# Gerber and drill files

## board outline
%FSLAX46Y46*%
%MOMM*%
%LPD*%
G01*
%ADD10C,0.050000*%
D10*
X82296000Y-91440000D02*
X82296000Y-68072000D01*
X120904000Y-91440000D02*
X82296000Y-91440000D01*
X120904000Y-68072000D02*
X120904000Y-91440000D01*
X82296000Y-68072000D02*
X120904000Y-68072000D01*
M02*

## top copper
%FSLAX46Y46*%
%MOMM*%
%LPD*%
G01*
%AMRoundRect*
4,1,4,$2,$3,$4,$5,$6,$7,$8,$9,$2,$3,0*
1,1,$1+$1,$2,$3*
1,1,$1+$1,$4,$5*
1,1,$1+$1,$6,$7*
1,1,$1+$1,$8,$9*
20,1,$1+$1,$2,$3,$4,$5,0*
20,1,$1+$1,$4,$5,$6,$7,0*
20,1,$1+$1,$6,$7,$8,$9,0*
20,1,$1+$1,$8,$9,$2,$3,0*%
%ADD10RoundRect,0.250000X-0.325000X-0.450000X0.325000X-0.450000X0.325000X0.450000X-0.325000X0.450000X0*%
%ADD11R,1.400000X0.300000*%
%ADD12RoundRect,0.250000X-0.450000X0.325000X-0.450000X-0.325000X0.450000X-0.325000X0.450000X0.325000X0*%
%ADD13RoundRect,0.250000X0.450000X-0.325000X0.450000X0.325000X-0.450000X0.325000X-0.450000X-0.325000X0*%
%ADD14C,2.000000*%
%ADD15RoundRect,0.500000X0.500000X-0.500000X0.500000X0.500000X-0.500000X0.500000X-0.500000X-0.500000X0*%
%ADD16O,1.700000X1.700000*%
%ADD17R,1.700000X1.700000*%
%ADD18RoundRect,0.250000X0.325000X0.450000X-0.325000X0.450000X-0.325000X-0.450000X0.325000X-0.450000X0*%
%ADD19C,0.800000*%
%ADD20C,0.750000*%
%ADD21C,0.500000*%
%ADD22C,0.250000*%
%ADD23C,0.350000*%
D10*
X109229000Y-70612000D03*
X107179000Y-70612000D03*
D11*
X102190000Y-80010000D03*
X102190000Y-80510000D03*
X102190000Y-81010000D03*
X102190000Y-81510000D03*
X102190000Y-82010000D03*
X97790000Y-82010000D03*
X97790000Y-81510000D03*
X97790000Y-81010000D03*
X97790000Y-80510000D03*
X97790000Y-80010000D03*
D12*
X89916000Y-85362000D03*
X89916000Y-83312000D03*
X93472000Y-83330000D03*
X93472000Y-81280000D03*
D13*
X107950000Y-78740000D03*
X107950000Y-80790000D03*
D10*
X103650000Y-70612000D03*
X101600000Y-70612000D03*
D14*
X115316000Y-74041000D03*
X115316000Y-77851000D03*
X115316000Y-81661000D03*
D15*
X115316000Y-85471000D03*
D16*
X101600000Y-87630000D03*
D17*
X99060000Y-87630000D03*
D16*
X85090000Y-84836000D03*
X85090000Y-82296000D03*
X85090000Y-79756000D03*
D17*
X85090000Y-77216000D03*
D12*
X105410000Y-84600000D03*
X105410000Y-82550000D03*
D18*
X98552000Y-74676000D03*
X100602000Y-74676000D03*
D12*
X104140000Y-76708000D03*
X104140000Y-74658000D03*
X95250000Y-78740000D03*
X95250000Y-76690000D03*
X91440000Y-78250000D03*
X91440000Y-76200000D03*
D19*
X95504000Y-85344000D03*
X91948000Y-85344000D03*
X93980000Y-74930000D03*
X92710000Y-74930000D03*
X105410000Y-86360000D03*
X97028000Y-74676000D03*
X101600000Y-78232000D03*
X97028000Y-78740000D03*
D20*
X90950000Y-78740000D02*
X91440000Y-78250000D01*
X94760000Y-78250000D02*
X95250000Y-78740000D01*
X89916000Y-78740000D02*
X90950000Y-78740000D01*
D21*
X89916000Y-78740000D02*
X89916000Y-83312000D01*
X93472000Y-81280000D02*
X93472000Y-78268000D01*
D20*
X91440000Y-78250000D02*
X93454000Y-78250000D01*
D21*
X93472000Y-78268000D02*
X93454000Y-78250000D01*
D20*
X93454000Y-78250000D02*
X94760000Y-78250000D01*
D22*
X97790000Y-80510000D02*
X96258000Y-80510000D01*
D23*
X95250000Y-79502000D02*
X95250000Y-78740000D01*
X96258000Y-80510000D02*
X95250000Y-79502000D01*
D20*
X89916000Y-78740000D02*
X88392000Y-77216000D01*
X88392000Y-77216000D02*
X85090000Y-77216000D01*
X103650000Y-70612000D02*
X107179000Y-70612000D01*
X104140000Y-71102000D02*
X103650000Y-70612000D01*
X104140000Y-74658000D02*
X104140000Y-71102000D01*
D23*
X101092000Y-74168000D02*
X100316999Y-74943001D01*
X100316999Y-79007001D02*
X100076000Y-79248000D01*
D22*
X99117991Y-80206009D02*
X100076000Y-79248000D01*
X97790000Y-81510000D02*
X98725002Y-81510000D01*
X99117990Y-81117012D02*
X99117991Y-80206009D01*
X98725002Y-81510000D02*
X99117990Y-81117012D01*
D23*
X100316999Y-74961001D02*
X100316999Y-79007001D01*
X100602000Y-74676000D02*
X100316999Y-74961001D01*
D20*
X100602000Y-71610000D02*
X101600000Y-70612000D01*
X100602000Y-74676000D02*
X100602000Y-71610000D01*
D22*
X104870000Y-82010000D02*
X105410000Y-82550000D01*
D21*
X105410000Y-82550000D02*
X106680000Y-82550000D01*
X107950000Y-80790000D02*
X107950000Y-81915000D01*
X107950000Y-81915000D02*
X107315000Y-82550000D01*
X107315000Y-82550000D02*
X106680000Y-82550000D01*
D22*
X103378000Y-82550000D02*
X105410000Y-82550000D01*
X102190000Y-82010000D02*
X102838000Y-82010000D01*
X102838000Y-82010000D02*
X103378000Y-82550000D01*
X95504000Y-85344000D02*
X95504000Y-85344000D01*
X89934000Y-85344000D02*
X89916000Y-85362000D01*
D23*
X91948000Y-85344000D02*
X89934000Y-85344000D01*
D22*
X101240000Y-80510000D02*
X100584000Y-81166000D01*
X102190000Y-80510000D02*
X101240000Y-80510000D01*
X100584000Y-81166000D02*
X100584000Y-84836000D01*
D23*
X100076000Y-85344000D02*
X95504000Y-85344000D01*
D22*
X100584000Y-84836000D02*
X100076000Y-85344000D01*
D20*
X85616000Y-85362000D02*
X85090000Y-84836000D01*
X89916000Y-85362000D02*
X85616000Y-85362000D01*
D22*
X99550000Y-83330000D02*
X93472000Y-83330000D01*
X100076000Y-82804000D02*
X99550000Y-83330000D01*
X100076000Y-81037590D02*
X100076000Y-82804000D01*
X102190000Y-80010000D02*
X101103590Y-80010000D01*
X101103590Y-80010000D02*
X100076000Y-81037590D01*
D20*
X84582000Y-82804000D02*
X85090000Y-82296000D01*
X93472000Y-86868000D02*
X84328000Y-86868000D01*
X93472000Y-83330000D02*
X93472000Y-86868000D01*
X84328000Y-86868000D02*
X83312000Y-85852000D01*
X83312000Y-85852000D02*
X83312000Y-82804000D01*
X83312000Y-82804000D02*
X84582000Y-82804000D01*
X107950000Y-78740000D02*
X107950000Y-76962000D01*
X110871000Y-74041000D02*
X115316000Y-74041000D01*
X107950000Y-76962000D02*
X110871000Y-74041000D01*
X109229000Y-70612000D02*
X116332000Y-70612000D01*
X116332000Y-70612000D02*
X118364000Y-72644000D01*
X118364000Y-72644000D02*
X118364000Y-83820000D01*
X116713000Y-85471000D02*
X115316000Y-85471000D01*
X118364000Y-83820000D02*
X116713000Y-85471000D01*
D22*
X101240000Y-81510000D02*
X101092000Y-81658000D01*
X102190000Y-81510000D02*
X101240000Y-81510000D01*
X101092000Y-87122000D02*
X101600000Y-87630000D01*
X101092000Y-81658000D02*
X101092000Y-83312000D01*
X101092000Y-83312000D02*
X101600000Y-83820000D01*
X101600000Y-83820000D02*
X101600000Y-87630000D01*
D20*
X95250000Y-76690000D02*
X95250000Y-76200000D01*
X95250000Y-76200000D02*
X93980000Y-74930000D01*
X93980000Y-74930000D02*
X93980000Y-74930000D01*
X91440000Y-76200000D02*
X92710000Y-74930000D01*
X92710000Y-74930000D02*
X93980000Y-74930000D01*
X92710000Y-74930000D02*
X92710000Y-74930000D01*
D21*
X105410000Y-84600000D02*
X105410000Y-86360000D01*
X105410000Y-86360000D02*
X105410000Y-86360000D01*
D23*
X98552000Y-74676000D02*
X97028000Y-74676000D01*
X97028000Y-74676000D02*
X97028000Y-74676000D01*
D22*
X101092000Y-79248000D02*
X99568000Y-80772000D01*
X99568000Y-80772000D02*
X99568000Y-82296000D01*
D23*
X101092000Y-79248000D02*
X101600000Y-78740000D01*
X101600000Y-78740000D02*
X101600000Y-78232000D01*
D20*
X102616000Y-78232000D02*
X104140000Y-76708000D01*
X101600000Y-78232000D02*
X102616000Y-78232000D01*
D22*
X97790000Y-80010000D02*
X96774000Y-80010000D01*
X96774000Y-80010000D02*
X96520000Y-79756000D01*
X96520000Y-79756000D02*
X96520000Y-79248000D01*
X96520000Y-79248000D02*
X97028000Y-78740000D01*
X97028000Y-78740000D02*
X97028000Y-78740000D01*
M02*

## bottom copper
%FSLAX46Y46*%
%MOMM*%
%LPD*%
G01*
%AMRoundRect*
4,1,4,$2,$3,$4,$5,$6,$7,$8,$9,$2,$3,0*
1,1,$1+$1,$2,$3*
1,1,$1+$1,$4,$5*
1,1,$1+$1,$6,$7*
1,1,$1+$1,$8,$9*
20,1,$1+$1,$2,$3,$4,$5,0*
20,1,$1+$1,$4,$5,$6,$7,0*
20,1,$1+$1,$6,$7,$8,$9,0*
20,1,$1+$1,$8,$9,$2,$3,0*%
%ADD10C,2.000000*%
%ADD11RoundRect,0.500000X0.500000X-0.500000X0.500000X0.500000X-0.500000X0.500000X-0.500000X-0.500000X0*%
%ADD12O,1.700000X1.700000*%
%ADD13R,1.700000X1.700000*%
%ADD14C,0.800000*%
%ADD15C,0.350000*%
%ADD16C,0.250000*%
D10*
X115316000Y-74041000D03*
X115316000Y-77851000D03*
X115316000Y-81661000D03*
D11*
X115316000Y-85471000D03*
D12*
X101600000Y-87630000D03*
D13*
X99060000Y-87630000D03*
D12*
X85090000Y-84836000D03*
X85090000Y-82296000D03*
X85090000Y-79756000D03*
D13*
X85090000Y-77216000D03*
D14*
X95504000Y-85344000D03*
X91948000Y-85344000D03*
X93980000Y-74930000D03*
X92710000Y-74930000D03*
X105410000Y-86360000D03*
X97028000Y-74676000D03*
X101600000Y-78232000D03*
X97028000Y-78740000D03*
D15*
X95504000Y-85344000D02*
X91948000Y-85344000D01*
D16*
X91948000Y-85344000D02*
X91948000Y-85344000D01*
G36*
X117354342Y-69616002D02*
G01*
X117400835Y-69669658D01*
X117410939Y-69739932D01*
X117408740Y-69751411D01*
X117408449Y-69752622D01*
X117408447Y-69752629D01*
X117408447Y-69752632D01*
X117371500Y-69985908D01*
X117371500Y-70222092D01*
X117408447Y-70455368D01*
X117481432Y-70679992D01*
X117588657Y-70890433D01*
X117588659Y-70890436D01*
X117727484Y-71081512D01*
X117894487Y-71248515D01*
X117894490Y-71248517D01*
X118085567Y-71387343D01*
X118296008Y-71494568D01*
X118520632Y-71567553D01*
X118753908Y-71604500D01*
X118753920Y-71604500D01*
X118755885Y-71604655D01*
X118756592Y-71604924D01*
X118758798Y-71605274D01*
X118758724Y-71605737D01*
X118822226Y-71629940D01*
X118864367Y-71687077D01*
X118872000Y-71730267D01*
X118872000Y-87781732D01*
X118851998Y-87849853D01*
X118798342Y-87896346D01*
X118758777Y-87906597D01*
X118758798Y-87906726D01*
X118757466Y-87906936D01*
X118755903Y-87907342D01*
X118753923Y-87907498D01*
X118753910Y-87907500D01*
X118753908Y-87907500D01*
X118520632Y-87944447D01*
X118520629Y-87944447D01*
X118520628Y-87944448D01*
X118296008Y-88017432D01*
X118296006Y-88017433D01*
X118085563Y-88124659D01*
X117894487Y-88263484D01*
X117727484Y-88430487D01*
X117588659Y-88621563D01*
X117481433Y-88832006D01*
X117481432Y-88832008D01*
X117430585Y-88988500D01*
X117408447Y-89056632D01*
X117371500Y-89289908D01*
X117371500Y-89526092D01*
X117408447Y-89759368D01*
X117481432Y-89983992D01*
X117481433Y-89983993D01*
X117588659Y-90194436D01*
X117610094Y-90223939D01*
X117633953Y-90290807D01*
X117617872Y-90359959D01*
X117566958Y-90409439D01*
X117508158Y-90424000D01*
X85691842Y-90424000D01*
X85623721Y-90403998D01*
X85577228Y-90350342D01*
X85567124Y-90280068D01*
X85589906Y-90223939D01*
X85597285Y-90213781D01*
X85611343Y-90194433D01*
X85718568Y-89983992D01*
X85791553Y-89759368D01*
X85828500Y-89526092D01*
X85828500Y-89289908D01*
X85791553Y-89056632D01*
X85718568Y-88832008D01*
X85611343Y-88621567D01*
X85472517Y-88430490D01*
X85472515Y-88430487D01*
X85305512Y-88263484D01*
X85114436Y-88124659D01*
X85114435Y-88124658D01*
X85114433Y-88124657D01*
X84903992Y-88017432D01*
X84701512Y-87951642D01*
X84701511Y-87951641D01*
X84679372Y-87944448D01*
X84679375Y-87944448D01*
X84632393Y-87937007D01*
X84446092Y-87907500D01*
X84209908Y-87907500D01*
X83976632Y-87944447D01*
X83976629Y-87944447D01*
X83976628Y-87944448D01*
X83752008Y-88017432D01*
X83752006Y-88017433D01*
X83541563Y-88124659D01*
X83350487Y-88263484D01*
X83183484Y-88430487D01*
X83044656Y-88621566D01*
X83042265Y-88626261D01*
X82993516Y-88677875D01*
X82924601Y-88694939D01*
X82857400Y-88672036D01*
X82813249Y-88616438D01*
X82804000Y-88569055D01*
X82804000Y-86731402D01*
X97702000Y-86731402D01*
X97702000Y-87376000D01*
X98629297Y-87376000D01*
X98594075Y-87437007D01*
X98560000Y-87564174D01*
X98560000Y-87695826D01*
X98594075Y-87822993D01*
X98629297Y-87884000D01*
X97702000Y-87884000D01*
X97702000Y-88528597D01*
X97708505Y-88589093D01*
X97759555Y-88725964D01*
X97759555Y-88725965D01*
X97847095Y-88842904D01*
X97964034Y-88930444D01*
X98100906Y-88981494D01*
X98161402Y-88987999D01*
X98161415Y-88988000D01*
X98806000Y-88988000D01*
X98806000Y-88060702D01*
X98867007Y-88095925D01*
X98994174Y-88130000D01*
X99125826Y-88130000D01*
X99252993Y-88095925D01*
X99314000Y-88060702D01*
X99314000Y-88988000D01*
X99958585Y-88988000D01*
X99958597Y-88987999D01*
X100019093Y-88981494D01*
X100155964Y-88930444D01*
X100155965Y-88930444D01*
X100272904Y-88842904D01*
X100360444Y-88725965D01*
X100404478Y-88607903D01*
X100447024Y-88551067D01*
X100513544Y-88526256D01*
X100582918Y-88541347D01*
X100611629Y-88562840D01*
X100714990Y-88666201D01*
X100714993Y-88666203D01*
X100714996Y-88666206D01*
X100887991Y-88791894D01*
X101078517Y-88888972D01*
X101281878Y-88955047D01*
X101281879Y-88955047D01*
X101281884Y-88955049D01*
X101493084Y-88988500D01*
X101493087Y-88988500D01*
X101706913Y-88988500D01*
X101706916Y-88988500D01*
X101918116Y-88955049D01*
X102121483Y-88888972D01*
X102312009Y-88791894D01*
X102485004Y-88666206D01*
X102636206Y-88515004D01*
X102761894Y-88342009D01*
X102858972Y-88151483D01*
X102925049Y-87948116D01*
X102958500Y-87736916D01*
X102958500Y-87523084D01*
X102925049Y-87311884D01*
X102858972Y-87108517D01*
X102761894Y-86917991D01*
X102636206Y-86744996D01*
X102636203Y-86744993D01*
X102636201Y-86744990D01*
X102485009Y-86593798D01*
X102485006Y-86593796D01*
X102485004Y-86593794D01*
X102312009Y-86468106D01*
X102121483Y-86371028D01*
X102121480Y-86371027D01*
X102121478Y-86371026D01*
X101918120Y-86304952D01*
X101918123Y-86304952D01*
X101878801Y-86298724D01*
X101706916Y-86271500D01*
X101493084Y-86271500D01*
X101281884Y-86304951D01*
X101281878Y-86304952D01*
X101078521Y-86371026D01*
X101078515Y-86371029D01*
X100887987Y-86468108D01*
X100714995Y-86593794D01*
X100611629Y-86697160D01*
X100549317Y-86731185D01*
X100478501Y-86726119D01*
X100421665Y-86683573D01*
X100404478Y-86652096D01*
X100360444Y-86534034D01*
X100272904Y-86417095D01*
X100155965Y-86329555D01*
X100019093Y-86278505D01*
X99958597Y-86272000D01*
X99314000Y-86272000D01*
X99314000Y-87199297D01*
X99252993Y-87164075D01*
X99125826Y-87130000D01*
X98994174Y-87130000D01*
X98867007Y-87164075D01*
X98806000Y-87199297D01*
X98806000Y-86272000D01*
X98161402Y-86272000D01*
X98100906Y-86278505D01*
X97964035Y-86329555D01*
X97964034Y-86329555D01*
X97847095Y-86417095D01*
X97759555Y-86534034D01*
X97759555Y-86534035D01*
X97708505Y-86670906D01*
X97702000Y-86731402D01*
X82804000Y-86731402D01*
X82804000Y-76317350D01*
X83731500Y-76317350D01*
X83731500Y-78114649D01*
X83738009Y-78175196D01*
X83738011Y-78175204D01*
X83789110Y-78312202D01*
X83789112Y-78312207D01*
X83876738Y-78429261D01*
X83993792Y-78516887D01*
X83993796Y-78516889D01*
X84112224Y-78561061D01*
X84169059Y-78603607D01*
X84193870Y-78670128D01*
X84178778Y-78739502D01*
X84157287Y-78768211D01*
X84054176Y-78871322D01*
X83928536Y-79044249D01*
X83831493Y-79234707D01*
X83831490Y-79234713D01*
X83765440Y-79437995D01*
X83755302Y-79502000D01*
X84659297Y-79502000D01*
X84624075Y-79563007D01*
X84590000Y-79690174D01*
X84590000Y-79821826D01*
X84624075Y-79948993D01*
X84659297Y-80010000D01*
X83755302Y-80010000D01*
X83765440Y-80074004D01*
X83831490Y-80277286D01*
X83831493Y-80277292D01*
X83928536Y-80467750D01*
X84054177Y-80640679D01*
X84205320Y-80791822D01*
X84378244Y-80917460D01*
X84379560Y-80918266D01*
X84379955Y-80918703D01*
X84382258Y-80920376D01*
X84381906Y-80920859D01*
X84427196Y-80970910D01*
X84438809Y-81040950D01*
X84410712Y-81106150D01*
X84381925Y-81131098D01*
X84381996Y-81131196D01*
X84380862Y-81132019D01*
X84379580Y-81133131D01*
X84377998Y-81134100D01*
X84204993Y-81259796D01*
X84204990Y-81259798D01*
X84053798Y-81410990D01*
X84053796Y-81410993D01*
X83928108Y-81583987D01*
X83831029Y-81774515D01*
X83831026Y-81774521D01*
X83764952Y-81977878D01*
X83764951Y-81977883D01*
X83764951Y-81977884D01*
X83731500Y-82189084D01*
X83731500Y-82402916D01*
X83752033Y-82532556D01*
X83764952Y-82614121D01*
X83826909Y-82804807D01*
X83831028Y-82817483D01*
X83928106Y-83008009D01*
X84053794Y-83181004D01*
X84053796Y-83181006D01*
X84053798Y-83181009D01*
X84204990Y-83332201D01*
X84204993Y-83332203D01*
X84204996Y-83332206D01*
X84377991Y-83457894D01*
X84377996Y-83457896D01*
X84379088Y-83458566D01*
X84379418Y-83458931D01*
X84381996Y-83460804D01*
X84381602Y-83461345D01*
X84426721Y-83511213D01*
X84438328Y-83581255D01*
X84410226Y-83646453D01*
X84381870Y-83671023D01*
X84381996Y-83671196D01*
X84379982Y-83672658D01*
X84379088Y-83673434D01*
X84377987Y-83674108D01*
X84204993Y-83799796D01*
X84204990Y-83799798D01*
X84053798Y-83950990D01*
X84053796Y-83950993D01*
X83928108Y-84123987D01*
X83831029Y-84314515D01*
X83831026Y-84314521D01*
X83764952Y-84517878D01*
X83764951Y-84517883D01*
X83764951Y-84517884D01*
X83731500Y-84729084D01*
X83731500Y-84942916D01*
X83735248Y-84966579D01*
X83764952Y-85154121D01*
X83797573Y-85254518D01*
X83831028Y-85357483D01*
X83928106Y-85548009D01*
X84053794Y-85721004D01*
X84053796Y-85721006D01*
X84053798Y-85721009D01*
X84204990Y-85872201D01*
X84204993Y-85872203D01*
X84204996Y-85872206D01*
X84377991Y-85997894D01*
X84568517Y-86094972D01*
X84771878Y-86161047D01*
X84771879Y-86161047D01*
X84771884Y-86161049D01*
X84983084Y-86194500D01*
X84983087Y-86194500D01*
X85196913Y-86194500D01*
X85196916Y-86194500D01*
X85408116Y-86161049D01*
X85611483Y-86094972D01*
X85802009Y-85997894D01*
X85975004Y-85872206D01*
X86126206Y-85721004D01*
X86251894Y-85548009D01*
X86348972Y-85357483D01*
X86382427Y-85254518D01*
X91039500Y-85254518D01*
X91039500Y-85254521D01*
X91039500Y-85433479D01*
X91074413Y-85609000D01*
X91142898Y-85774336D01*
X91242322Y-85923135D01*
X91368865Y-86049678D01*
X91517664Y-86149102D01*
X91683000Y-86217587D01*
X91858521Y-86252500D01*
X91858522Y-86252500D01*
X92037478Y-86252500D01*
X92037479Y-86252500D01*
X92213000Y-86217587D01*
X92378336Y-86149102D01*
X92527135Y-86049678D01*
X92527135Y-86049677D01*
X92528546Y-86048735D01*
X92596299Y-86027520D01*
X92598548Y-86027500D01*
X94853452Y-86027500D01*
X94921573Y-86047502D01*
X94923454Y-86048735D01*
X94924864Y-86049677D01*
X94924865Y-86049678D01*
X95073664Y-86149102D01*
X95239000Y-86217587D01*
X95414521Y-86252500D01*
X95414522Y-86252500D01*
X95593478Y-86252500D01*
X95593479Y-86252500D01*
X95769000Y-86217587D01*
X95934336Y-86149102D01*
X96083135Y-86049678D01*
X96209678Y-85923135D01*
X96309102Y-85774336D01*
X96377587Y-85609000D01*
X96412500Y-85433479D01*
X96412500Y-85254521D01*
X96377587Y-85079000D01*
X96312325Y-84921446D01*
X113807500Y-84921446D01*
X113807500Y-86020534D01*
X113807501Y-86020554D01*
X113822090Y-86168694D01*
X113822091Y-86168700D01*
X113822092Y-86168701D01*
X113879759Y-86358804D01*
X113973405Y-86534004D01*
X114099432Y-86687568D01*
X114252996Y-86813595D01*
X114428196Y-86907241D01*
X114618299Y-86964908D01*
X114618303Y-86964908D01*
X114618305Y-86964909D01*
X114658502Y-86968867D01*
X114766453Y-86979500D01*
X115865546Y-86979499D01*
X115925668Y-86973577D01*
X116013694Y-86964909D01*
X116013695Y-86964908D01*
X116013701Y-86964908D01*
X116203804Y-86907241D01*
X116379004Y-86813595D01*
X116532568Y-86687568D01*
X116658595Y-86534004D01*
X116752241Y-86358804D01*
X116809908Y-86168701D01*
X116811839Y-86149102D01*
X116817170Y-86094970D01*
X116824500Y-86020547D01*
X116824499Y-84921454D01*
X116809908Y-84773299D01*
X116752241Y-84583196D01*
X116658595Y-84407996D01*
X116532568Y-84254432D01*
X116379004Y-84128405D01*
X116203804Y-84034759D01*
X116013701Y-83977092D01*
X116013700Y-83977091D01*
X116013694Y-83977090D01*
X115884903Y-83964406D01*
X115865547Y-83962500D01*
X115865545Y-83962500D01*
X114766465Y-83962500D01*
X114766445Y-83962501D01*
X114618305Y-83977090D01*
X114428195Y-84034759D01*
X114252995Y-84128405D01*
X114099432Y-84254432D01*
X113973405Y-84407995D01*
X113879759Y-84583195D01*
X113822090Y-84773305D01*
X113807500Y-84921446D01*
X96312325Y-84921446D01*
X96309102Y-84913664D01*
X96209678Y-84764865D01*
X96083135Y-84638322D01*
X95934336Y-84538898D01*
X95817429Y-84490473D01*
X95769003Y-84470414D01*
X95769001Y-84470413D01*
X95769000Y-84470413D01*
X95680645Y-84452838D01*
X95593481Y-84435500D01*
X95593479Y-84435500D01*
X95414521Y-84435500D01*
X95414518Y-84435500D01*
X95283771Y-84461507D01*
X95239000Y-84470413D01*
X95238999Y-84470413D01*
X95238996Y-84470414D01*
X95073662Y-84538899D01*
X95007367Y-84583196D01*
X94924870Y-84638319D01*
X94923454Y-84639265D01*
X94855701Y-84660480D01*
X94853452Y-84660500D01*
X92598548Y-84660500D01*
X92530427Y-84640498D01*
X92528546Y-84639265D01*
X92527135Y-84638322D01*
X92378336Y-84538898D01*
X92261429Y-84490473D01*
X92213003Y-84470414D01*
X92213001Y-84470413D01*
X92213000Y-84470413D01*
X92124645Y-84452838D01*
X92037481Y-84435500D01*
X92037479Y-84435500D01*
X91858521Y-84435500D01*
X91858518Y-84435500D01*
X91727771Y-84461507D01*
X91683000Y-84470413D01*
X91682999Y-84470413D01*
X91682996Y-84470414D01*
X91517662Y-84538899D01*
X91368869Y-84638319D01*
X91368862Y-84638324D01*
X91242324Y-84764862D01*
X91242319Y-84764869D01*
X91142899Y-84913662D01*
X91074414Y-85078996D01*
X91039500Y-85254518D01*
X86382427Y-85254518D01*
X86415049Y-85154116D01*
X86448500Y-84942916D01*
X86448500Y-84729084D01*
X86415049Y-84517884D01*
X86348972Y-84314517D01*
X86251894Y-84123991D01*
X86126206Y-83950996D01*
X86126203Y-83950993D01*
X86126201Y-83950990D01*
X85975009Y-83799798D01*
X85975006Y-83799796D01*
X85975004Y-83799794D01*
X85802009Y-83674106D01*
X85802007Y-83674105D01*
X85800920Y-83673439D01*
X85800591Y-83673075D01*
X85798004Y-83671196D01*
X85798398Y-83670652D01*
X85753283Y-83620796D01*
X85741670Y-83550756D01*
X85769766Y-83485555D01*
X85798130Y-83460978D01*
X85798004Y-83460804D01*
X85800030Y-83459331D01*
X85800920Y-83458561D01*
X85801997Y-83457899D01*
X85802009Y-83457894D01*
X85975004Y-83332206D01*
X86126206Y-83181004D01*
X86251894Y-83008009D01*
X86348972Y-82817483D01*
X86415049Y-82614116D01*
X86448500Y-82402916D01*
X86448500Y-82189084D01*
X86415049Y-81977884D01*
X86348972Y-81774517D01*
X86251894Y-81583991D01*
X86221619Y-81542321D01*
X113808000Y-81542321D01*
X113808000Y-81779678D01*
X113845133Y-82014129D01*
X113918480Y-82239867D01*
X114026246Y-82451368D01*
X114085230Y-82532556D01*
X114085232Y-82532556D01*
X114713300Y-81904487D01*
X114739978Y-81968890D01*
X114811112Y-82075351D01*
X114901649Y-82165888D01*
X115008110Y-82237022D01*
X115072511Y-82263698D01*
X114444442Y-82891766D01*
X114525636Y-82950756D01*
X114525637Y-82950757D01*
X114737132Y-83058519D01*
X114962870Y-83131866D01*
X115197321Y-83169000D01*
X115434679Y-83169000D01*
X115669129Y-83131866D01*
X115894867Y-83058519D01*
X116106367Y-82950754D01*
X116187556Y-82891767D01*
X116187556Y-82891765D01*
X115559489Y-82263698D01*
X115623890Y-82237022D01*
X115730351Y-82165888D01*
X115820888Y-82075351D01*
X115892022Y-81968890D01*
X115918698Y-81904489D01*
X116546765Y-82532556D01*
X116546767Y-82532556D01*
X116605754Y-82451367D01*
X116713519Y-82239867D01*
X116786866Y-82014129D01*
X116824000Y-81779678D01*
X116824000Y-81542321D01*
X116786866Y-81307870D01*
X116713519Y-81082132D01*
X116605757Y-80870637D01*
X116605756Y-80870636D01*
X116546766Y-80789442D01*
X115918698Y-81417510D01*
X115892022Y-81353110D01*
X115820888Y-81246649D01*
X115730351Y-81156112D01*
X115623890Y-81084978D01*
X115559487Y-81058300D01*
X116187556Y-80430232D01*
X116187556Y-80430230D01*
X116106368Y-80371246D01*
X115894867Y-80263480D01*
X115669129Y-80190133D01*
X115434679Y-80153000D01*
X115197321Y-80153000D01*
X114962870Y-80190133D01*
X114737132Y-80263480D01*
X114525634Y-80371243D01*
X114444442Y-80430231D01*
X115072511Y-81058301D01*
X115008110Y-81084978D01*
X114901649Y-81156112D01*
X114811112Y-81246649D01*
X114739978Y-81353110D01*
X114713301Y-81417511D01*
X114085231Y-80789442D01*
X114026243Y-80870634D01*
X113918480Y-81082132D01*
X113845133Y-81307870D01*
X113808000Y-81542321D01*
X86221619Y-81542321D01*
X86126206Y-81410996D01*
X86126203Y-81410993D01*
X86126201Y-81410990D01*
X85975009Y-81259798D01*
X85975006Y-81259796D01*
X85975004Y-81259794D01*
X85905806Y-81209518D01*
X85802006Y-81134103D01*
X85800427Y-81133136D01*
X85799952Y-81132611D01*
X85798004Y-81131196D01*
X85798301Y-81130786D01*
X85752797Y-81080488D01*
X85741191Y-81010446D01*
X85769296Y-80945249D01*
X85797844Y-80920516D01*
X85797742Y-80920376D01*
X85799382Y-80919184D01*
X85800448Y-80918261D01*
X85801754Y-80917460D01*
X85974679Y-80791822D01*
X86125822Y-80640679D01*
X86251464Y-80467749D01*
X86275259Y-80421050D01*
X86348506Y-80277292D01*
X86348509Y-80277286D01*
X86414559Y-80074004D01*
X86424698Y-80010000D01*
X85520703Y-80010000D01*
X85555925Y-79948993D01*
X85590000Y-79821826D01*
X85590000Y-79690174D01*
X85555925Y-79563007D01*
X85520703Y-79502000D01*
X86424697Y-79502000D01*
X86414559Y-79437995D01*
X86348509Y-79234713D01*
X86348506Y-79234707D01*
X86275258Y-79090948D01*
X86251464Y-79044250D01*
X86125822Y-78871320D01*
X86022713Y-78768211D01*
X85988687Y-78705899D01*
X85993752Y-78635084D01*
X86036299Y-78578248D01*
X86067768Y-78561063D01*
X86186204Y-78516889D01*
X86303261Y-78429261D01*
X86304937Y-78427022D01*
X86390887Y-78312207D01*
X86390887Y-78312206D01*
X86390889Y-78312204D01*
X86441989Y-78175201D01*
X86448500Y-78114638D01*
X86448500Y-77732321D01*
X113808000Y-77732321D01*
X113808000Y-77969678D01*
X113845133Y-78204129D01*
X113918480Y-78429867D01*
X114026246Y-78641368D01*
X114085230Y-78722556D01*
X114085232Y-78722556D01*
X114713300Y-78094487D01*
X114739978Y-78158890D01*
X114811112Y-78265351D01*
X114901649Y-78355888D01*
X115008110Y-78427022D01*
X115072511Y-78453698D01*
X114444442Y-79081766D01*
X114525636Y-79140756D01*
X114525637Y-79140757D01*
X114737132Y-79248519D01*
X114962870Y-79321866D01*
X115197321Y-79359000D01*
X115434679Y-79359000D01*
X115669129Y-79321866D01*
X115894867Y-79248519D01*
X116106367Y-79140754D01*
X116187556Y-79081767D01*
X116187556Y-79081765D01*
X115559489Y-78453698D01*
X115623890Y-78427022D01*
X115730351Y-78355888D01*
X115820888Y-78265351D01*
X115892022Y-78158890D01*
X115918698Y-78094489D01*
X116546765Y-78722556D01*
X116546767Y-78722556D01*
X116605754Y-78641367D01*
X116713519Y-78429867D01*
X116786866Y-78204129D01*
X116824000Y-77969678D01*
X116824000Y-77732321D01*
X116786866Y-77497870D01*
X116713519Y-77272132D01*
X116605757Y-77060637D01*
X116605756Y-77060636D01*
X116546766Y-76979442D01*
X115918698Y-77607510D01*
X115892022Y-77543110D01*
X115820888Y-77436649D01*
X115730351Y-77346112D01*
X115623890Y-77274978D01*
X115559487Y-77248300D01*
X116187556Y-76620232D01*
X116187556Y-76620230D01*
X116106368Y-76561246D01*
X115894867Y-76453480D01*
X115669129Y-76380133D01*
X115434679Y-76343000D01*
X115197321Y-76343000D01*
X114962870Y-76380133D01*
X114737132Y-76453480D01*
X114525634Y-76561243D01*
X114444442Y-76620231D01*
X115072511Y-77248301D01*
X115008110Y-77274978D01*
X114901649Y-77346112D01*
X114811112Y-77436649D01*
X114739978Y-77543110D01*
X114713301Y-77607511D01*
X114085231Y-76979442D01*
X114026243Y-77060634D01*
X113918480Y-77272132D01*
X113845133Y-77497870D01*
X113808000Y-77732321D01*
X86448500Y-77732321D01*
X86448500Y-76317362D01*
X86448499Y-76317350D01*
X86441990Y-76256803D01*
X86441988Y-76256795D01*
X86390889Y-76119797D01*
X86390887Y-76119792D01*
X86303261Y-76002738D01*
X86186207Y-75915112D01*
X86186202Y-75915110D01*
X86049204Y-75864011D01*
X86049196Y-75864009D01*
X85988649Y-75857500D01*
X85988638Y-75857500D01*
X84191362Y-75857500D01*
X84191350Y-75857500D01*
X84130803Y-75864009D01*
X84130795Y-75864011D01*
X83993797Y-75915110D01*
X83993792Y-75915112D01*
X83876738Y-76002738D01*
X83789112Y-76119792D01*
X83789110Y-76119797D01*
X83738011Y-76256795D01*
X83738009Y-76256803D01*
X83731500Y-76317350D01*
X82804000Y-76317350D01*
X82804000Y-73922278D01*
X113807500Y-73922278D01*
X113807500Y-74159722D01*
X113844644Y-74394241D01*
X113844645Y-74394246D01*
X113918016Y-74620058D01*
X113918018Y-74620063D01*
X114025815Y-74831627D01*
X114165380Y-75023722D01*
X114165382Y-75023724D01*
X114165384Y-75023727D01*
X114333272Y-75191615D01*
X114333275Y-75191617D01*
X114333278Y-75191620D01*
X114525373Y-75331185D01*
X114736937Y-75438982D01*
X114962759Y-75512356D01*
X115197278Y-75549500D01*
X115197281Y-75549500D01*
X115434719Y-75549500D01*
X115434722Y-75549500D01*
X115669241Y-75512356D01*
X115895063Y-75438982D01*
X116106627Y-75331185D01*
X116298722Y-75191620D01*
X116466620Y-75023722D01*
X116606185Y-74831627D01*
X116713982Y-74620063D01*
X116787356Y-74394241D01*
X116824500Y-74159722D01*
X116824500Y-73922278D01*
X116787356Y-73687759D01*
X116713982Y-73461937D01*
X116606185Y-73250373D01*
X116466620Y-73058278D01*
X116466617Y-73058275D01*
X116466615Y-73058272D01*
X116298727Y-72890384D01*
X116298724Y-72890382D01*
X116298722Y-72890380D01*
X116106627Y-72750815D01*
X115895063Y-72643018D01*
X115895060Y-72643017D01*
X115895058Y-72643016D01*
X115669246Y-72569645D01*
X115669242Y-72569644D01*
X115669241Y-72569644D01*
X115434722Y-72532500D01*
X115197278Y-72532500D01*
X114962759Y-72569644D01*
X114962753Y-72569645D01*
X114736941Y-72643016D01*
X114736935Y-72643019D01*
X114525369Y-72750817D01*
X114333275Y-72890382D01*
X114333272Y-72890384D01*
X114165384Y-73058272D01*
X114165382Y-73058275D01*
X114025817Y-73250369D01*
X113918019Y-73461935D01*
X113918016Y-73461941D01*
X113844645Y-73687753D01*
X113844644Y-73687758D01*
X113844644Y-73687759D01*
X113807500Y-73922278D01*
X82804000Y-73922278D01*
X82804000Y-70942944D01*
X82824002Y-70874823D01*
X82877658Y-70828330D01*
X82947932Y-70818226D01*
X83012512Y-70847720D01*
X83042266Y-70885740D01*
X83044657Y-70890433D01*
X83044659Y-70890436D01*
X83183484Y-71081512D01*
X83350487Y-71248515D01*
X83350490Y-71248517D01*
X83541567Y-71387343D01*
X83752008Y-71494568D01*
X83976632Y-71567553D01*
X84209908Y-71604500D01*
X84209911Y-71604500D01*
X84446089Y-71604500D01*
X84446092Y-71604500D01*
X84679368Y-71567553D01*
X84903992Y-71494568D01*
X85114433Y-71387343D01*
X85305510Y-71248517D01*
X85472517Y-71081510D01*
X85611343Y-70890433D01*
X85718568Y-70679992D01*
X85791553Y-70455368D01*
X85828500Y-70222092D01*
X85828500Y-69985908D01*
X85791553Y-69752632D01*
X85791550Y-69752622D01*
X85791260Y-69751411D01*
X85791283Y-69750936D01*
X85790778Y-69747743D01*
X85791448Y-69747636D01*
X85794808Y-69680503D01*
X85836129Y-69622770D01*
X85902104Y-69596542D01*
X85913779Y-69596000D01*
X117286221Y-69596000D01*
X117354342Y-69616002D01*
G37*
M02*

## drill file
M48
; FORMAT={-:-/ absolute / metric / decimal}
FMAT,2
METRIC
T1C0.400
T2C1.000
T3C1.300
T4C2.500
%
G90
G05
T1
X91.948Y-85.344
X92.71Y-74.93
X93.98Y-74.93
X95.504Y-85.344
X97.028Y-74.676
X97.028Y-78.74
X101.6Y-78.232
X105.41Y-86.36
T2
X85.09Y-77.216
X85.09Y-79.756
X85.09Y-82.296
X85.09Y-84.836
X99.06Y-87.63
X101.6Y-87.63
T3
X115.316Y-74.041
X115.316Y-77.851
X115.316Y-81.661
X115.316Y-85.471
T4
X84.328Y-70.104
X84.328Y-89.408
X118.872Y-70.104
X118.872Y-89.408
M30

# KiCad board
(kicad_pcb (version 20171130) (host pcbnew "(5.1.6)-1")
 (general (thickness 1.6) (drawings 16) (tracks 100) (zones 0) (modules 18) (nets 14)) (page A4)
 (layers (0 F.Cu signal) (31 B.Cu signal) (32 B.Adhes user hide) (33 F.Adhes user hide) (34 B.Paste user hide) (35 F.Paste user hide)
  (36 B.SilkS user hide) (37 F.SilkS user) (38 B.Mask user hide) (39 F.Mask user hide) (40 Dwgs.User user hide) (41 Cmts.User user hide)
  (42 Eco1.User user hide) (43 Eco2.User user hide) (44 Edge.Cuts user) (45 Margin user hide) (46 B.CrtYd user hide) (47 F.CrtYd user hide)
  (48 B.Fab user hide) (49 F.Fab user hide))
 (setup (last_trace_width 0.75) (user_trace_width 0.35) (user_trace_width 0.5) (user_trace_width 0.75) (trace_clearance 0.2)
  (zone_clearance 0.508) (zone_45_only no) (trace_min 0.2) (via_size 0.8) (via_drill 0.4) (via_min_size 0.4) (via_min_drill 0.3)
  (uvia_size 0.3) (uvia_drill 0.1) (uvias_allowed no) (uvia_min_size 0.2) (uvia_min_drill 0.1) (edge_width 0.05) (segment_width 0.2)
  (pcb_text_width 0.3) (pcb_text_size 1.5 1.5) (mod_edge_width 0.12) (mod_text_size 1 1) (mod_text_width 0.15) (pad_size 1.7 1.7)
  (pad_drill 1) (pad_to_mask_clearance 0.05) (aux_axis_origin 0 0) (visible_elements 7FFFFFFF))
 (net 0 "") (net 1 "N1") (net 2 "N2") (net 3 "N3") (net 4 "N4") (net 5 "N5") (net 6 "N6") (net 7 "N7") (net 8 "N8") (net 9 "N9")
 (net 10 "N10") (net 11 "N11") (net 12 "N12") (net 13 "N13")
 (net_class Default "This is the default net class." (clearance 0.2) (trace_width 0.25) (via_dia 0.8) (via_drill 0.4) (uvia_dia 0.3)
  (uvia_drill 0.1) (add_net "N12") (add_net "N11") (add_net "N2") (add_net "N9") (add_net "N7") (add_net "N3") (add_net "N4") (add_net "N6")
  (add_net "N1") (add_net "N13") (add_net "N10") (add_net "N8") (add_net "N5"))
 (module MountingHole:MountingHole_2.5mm (layer F.Cu) (at 84.328 89.408)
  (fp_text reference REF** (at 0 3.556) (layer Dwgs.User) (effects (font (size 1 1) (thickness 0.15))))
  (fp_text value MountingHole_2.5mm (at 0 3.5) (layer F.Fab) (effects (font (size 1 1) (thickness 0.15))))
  (pad 1 np_thru_hole circle (at 0 0) (size 2.5 2.5) (drill 2.5) (layers *.Cu *.Mask)))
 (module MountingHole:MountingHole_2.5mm (layer F.Cu) (at 118.872 89.408)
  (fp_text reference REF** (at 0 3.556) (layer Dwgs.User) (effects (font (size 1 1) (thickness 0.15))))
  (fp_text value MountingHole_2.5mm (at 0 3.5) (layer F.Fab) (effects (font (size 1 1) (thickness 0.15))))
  (pad 1 np_thru_hole circle (at 0 0) (size 2.5 2.5) (drill 2.5) (layers *.Cu *.Mask)))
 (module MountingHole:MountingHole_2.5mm (layer F.Cu) (at 118.872 70.104)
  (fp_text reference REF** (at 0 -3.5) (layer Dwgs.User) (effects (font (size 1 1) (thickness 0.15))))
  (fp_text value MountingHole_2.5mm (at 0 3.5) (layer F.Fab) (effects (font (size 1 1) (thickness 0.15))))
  (pad 1 np_thru_hole circle (at 0 0) (size 2.5 2.5) (drill 2.5) (layers *.Cu *.Mask)))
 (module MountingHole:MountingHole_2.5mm (layer F.Cu) (at 84.328 70.104)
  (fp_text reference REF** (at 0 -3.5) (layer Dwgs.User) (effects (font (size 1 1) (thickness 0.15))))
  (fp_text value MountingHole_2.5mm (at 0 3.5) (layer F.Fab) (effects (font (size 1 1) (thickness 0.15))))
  (pad 1 np_thru_hole circle (at 0 0) (size 2.5 2.5) (drill 2.5) (layers *.Cu *.Mask)))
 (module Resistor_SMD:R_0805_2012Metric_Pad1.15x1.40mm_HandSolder (layer F.Cu) (at 108.204 70.612)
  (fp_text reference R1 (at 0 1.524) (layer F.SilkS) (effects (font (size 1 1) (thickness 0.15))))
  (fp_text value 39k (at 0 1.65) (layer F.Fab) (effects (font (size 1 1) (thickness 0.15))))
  (pad 2 smd roundrect (at 1.025 0) (size 1.15 1.4) (layers F.Cu F.Paste F.Mask) (roundrect_rratio 0.217391) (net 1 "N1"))
  (pad 1 smd roundrect (at -1.025 0) (size 1.15 1.4) (layers F.Cu F.Paste F.Mask) (roundrect_rratio 0.217391) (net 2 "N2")))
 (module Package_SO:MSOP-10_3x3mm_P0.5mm (layer F.Cu) (at 99.99 81.01)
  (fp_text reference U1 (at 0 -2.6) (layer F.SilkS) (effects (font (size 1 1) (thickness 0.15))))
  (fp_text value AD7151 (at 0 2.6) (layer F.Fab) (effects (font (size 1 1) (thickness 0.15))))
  (pad 10 smd rect (at 2.2 -1) (size 1.4 0.3) (layers F.Cu F.Paste F.Mask) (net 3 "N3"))
  (pad 9 smd rect (at 2.2 -0.5) (size 1.4 0.3) (layers F.Cu F.Paste F.Mask) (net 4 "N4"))
  (pad 8 smd rect (at 2.2 0) (size 1.4 0.3) (layers F.Cu F.Paste F.Mask) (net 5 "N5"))
  (pad 7 smd rect (at 2.2 0.5) (size 1.4 0.3) (layers F.Cu F.Paste F.Mask) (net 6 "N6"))
  (pad 6 smd rect (at 2.2 1) (size 1.4 0.3) (layers F.Cu F.Paste F.Mask) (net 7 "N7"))
  (pad 5 smd rect (at -2.2 1) (size 1.4 0.3) (layers F.Cu F.Paste F.Mask) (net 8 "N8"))
  (pad 4 smd rect (at -2.2 0.5) (size 1.4 0.3) (layers F.Cu F.Paste F.Mask) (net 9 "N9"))
  (pad 3 smd rect (at -2.2 0) (size 1.4 0.3) (layers F.Cu F.Paste F.Mask) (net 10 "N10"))
  (pad 2 smd rect (at -2.2 -0.5) (size 1.4 0.3) (layers F.Cu F.Paste F.Mask) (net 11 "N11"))
  (pad 1 smd rect (at -2.2 -1) (size 1.4 0.3) (layers F.Cu F.Paste F.Mask) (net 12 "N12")))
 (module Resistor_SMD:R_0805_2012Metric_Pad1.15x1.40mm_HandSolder (layer F.Cu) (at 89.916 84.337 270)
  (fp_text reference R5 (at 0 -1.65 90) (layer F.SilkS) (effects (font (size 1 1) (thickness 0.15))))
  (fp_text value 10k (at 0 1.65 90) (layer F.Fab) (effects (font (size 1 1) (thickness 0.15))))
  (pad 2 smd roundrect (at 1.025 0 270) (size 1.15 1.4) (layers F.Cu F.Paste F.Mask) (roundrect_rratio 0.217391) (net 4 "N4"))
  (pad 1 smd roundrect (at -1.025 0 270) (size 1.15 1.4) (layers F.Cu F.Paste F.Mask) (roundrect_rratio 0.217391) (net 11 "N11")))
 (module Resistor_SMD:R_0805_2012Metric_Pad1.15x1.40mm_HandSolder (layer F.Cu) (at 93.472 82.305 270)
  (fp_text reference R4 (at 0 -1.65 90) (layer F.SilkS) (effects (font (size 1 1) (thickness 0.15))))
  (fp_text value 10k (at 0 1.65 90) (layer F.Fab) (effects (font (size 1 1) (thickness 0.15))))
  (pad 2 smd roundrect (at 1.025 0 270) (size 1.15 1.4) (layers F.Cu F.Paste F.Mask) (roundrect_rratio 0.217391) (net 3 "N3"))
  (pad 1 smd roundrect (at -1.025 0 270) (size 1.15 1.4) (layers F.Cu F.Paste F.Mask) (roundrect_rratio 0.217391) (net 11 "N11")))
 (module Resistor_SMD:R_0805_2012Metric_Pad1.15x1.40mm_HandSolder (layer F.Cu) (at 107.95 79.765 90)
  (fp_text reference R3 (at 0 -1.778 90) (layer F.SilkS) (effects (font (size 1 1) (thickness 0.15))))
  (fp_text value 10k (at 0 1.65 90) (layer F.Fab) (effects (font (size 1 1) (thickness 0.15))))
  (pad 2 smd roundrect (at 1.025 0 90) (size 1.15 1.4) (layers F.Cu F.Paste F.Mask) (roundrect_rratio 0.217391) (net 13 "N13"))
  (pad 1 smd roundrect (at -1.025 0 90) (size 1.15 1.4) (layers F.Cu F.Paste F.Mask) (roundrect_rratio 0.217391) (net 7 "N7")))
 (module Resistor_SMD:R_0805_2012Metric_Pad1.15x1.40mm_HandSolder (layer F.Cu) (at 102.625 70.612)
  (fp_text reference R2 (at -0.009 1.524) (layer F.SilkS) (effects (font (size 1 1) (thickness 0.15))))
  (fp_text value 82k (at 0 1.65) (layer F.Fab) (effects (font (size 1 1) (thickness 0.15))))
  (pad 2 smd roundrect (at 1.025 0) (size 1.15 1.4) (layers F.Cu F.Paste F.Mask) (roundrect_rratio 0.217391) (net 2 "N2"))
  (pad 1 smd roundrect (at -1.025 0) (size 1.15 1.4) (layers F.Cu F.Paste F.Mask) (roundrect_rratio 0.217391) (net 9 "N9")))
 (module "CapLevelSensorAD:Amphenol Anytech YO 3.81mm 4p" (layer F.Cu) (at 115.316 79.756 90)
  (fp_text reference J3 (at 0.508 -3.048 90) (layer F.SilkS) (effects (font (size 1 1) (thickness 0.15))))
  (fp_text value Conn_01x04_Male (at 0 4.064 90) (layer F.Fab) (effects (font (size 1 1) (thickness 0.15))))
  (pad 4 thru_hole circle (at 5.715 0 90) (size 2 2) (drill 1.3) (layers *.Cu *.Mask) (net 13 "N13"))
  (pad 3 thru_hole circle (at 1.905 0 90) (size 2 2) (drill 1.3) (layers *.Cu *.Mask) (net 12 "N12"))
  (pad 2 thru_hole circle (at -1.905 0 90) (size 2 2) (drill 1.3) (layers *.Cu *.Mask) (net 12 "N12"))
  (pad 1 thru_hole roundrect (at -5.715 0 90) (size 2 2) (drill 1.3) (layers *.Cu *.Mask) (roundrect_rratio 0.25) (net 1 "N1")))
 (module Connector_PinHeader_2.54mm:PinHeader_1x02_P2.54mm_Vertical (layer F.Cu) (at 99.06 87.63 90)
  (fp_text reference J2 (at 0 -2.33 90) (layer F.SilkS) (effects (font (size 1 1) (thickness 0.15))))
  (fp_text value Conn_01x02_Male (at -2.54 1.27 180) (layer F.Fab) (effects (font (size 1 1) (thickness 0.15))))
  (pad 2 thru_hole oval (at 0 2.54 90) (size 1.7 1.7) (drill 1) (layers *.Cu *.Mask) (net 6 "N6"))
  (pad 1 thru_hole rect (at 0 0 90) (size 1.7 1.7) (drill 1) (layers *.Cu *.Mask) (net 12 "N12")))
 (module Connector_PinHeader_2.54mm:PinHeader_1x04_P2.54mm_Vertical (layer F.Cu) (at 85.09 77.216)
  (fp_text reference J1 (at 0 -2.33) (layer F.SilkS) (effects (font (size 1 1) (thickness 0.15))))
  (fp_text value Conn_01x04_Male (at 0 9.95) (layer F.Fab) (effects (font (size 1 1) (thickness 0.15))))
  (pad 4 thru_hole oval (at 0 7.62) (size 1.7 1.7) (drill 1) (layers *.Cu *.Mask) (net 4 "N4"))
  (pad 3 thru_hole oval (at 0 5.08) (size 1.7 1.7) (drill 1) (layers *.Cu *.Mask) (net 3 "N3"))
  (pad 2 thru_hole oval (at 0 2.54) (size 1.7 1.7) (drill 1) (layers *.Cu *.Mask) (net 12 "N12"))
  (pad 1 thru_hole rect (at 0 0) (size 1.7 1.7) (drill 1) (layers *.Cu *.Mask) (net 11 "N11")))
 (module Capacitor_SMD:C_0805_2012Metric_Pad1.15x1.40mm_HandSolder (layer F.Cu) (at 105.41 83.575 270)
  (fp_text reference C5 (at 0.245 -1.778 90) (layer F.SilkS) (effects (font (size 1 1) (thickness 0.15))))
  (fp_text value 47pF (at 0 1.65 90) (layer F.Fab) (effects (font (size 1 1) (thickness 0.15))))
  (pad 2 smd roundrect (at 1.025 0 270) (size 1.15 1.4) (layers F.Cu F.Paste F.Mask) (roundrect_rratio 0.217391) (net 12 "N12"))
  (pad 1 smd roundrect (at -1.025 0 270) (size 1.15 1.4) (layers F.Cu F.Paste F.Mask) (roundrect_rratio 0.217391) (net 7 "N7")))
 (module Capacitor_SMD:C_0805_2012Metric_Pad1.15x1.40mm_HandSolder (layer F.Cu) (at 99.577 74.676 180)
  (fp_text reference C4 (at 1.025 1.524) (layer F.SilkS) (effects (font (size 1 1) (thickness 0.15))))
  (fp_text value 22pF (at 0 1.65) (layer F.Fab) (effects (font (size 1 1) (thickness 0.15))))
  (pad 2 smd roundrect (at 1.025 0 180) (size 1.15 1.4) (layers F.Cu F.Paste F.Mask) (roundrect_rratio 0.217391) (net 12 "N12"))
  (pad 1 smd roundrect (at -1.025 0 180) (size 1.15 1.4) (layers F.Cu F.Paste F.Mask) (roundrect_rratio 0.217391) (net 9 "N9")))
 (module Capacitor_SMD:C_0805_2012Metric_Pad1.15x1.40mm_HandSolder (layer F.Cu) (at 104.14 75.683 270)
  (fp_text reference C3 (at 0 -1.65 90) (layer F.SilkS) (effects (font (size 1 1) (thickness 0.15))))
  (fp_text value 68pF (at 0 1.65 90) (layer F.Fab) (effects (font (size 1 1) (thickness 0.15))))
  (pad 2 smd roundrect (at 1.025 0 270) (size 1.15 1.4) (layers F.Cu F.Paste F.Mask) (roundrect_rratio 0.217391) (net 12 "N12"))
  (pad 1 smd roundrect (at -1.025 0 270) (size 1.15 1.4) (layers F.Cu F.Paste F.Mask) (roundrect_rratio 0.217391) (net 2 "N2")))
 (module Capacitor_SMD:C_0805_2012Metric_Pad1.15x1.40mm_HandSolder (layer F.Cu) (at 95.25 77.715 270)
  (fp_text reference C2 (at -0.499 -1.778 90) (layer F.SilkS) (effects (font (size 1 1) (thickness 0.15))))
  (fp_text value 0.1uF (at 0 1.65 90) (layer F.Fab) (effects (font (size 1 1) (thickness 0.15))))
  (pad 2 smd roundrect (at 1.025 0 270) (size 1.15 1.4) (layers F.Cu F.Paste F.Mask) (roundrect_rratio 0.217391) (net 11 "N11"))
  (pad 1 smd roundrect (at -1.025 0 270) (size 1.15 1.4) (layers F.Cu F.Paste F.Mask) (roundrect_rratio 0.217391) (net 12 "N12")))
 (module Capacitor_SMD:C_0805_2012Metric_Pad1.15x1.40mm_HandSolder (layer F.Cu) (at 91.44 77.225 270)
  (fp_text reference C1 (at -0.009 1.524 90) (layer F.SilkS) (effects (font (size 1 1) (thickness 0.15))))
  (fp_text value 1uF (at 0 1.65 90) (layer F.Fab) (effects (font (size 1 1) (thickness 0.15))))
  (pad 2 smd roundrect (at 1.025 0 270) (size 1.15 1.4) (layers F.Cu F.Paste F.Mask) (roundrect_rratio 0.217391) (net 11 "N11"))
  (pad 1 smd roundrect (at -1.025 0 270) (size 1.15 1.4) (layers F.Cu F.Paste F.Mask) (roundrect_rratio 0.217391) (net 12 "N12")))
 (gr_line (start 82.296 91.44) (end 82.296 68.072) (layer Edge.Cuts) (width 0.05))
 (gr_line (start 120.904 91.44) (end 82.296 91.44) (layer Edge.Cuts) (width 0.05))
 (gr_line (start 120.904 68.072) (end 120.904 91.44) (layer Edge.Cuts) (width 0.05))
 (gr_line (start 82.296 68.072) (end 120.904 68.072) (layer Edge.Cuts) (width 0.05))
 (segment (start 90.95 78.74) (end 91.44 78.25) (width 0.75) (layer F.Cu) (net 11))
 (segment (start 94.76 78.25) (end 95.25 78.74) (width 0.75) (layer F.Cu) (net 11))
 (segment (start 89.916 78.74) (end 90.95 78.74) (width 0.75) (layer F.Cu) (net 11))
 (segment (start 89.916 78.74) (end 89.916 83.312) (width 0.5) (layer F.Cu) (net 11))
 (segment (start 93.472 81.28) (end 93.472 78.268) (width 0.5) (layer F.Cu) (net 11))
 (segment (start 91.44 78.25) (end 93.454 78.25) (width 0.75) (layer F.Cu) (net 11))
 (segment (start 93.472 78.268) (end 93.454 78.25) (width 0.5) (layer F.Cu) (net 11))
 (segment (start 93.454 78.25) (end 94.76 78.25) (width 0.75) (layer F.Cu) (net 11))
 (segment (start 97.79 80.51) (end 96.258 80.51) (width 0.25) (layer F.Cu) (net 11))
 (segment (start 95.25 79.502) (end 95.25 78.74) (width 0.35) (layer F.Cu) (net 11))
 (segment (start 96.258 80.51) (end 95.25 79.502) (width 0.35) (layer F.Cu) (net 11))
 (segment (start 89.916 78.74) (end 88.392 77.216) (width 0.75) (layer F.Cu) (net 11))
 (segment (start 88.392 77.216) (end 85.09 77.216) (width 0.75) (layer F.Cu) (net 11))
 (segment (start 103.65 70.612) (end 107.179 70.612) (width 0.75) (layer F.Cu) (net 2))
 (segment (start 104.14 71.102) (end 103.65 70.612) (width 0.75) (layer F.Cu) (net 2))
 (segment (start 104.14 74.658) (end 104.14 71.102) (width 0.75) (layer F.Cu) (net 2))
 (segment (start 101.092 74.168) (end 100.316999 74.943001) (width 0.35) (layer F.Cu) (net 9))
 (segment (start 100.316999 79.007001) (end 100.076 79.248) (width 0.35) (layer F.Cu) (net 9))
 (segment (start 99.117991 80.206009) (end 100.076 79.248) (width 0.25) (layer F.Cu) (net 9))
 (segment (start 97.79 81.51) (end 98.725002 81.51) (width 0.25) (layer F.Cu) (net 9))
 (segment (start 99.11799 81.117012) (end 99.117991 80.206009) (width 0.25) (layer F.Cu) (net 9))
 (segment (start 98.725002 81.51) (end 99.11799 81.117012) (width 0.25) (layer F.Cu) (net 9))
 (segment (start 100.316999 74.961001) (end 100.316999 79.007001) (width 0.35) (layer F.Cu) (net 9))
 (segment (start 100.602 74.676) (end 100.316999 74.961001) (width 0.35) (layer F.Cu) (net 9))
 (segment (start 100.602 71.61) (end 101.6 70.612) (width 0.75) (layer F.Cu) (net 9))
 (segment (start 100.602 74.676) (end 100.602 71.61) (width 0.75) (layer F.Cu) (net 9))
 (segment (start 104.87 82.01) (end 105.41 82.55) (width 0.25) (layer F.Cu) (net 7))
 (segment (start 105.41 82.55) (end 106.68 82.55) (width 0.5) (layer F.Cu) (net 7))
 (segment (start 107.95 80.79) (end 107.95 81.915) (width 0.5) (layer F.Cu) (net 7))
 (segment (start 107.95 81.915) (end 107.315 82.55) (width 0.5) (layer F.Cu) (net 7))
 (segment (start 107.315 82.55) (end 106.68 82.55) (width 0.5) (layer F.Cu) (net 7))
 (segment (start 103.378 82.55) (end 105.41 82.55) (width 0.25) (layer F.Cu) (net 7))
 (segment (start 102.19 82.01) (end 102.838 82.01) (width 0.25) (layer F.Cu) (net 7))
 (segment (start 102.838 82.01) (end 103.378 82.55) (width 0.25) (layer F.Cu) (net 7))
 (segment (start 95.504 85.344) (end 95.504 85.344) (width 0.25) (layer F.Cu) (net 4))
 (via (at 95.504 85.344) (size 0.8) (drill 0.4) (layers F.Cu B.Cu) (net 4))
 (segment (start 95.504 85.344) (end 91.948 85.344) (width 0.35) (layer B.Cu) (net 4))
 (segment (start 91.948 85.344) (end 91.948 85.344) (width 0.25) (layer B.Cu) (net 4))
 (via (at 91.948 85.344) (size 0.8) (drill 0.4) (layers F.Cu B.Cu) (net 4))
 (segment (start 89.934 85.344) (end 89.916 85.362) (width 0.25) (layer F.Cu) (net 4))
 (segment (start 91.948 85.344) (end 89.934 85.344) (width 0.35) (layer F.Cu) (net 4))
 (segment (start 101.24 80.51) (end 100.584 81.166) (width 0.25) (layer F.Cu) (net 4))
 (segment (start 102.19 80.51) (end 101.24 80.51) (width 0.25) (layer F.Cu) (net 4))
 (segment (start 100.584 81.166) (end 100.584 84.836) (width 0.25) (layer F.Cu) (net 4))
 (segment (start 100.076 85.344) (end 95.504 85.344) (width 0.35) (layer F.Cu) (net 4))
 (segment (start 100.584 84.836) (end 100.076 85.344) (width 0.25) (layer F.Cu) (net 4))
 (segment (start 85.616 85.362) (end 85.09 84.836) (width 0.75) (layer F.Cu) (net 4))
 (segment (start 89.916 85.362) (end 85.616 85.362) (width 0.75) (layer F.Cu) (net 4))
 (segment (start 99.55 83.33) (end 93.472 83.33) (width 0.25) (layer F.Cu) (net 3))
 (segment (start 100.076 82.804) (end 99.55 83.33) (width 0.25) (layer F.Cu) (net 3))
 (segment (start 100.076 81.03759) (end 100.076 82.804) (width 0.25) (layer F.Cu) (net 3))
 (segment (start 102.19 80.01) (end 101.10359 80.01) (width 0.25) (layer F.Cu) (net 3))
 (segment (start 101.10359 80.01) (end 100.076 81.03759) (width 0.25) (layer F.Cu) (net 3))
 (segment (start 84.582 82.804) (end 85.09 82.296) (width 0.75) (layer F.Cu) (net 3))
 (segment (start 93.472 86.868) (end 84.328 86.868) (width 0.75) (layer F.Cu) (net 3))
 (segment (start 93.472 83.33) (end 93.472 86.868) (width 0.75) (layer F.Cu) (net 3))
 (segment (start 84.328 86.868) (end 83.312 85.852) (width 0.75) (layer F.Cu) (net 3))
 (segment (start 83.312 85.852) (end 83.312 82.804) (width 0.75) (layer F.Cu) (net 3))
 (segment (start 83.312 82.804) (end 84.582 82.804) (width 0.75) (layer F.Cu) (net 3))
 (segment (start 107.95 78.74) (end 107.95 76.962) (width 0.75) (layer F.Cu) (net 13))
 (segment (start 110.871 74.041) (end 115.316 74.041) (width 0.75) (layer F.Cu) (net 13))
 (segment (start 107.95 76.962) (end 110.871 74.041) (width 0.75) (layer F.Cu) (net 13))
 (segment (start 109.229 70.612) (end 116.332 70.612) (width 0.75) (layer F.Cu) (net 1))
 (segment (start 116.332 70.612) (end 118.364 72.644) (width 0.75) (layer F.Cu) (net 1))
 (segment (start 118.364 72.644) (end 118.364 83.82) (width 0.75) (layer F.Cu) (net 1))
 (segment (start 116.713 85.471) (end 115.316 85.471) (width 0.75) (layer F.Cu) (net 1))
 (segment (start 118.364 83.82) (end 116.713 85.471) (width 0.75) (layer F.Cu) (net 1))
 (segment (start 101.24 81.51) (end 101.092 81.658) (width 0.25) (layer F.Cu) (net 6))
 (segment (start 102.19 81.51) (end 101.24 81.51) (width 0.25) (layer F.Cu) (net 6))
 (segment (start 101.092 87.122) (end 101.6 87.63) (width 0.25) (layer F.Cu) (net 6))
 (segment (start 101.092 81.658) (end 101.092 83.312) (width 0.25) (layer F.Cu) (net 6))
 (segment (start 101.092 83.312) (end 101.6 83.82) (width 0.25) (layer F.Cu) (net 6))
 (segment (start 101.6 83.82) (end 101.6 87.63) (width 0.25) (layer F.Cu) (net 6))
 (segment (start 95.25 76.69) (end 95.25 76.2) (width 0.75) (layer F.Cu) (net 12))
 (segment (start 95.25 76.2) (end 93.98 74.93) (width 0.75) (layer F.Cu) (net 12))
 (segment (start 93.98 74.93) (end 93.98 74.93) (width 0.75) (layer F.Cu) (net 12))
 (via (at 93.98 74.93) (size 0.8) (drill 0.4) (layers F.Cu B.Cu) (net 12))
 (segment (start 91.44 76.2) (end 92.71 74.93) (width 0.75) (layer F.Cu) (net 12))
 (segment (start 92.71 74.93) (end 93.98 74.93) (width 0.75) (layer F.Cu) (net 12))
 (segment (start 92.71 74.93) (end 92.71 74.93) (width 0.75) (layer F.Cu) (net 12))
 (via (at 92.71 74.93) (size 0.8) (drill 0.4) (layers F.Cu B.Cu) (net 12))
 (segment (start 105.41 84.6) (end 105.41 86.36) (width 0.5) (layer F.Cu) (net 12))
 (segment (start 105.41 86.36) (end 105.41 86.36) (width 0.5) (layer F.Cu) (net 12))
 (via (at 105.41 86.36) (size 0.8) (drill 0.4) (layers F.Cu B.Cu) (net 12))
 (segment (start 98.552 74.676) (end 97.028 74.676) (width 0.35) (layer F.Cu) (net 12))
 (segment (start 97.028 74.676) (end 97.028 74.676) (width 0.35) (layer F.Cu) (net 12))
 (via (at 97.028 74.676) (size 0.8) (drill 0.4) (layers F.Cu B.Cu) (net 12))
 (via (at 101.6 78.232) (size 0.8) (drill 0.4) (layers F.Cu B.Cu) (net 12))
 (segment (start 101.092 79.248) (end 99.568 80.772) (width 0.25) (layer F.Cu) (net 12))
 (segment (start 99.568 80.772) (end 99.568 82.296) (width 0.25) (layer F.Cu) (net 12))
 (segment (start 101.092 79.248) (end 101.6 78.74) (width 0.35) (layer F.Cu) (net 12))
 (segment (start 101.6 78.74) (end 101.6 78.232) (width 0.35) (layer F.Cu) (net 12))
 (segment (start 102.616 78.232) (end 104.14 76.708) (width 0.75) (layer F.Cu) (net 12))
 (segment (start 101.6 78.232) (end 102.616 78.232) (width 0.75) (layer F.Cu) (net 12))
 (segment (start 97.79 80.01) (end 96.774 80.01) (width 0.25) (layer F.Cu) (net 12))
 (segment (start 96.774 80.01) (end 96.52 79.756) (width 0.25) (layer F.Cu) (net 12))
 (segment (start 96.52 79.756) (end 96.52 79.248) (width 0.25) (layer F.Cu) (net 12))
 (segment (start 96.52 79.248) (end 97.028 78.74) (width 0.25) (layer F.Cu) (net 12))
 (segment (start 97.028 78.74) (end 97.028 78.74) (width 0.25) (layer F.Cu) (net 12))
 (via (at 97.028 78.74) (size 0.8) (drill 0.4) (layers F.Cu B.Cu) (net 12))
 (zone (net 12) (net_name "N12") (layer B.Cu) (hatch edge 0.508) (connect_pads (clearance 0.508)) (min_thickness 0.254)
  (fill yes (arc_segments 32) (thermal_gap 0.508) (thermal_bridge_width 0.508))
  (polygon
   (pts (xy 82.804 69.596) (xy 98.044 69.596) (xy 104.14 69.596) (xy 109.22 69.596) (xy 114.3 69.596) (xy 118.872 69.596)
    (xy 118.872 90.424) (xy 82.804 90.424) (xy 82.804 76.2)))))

